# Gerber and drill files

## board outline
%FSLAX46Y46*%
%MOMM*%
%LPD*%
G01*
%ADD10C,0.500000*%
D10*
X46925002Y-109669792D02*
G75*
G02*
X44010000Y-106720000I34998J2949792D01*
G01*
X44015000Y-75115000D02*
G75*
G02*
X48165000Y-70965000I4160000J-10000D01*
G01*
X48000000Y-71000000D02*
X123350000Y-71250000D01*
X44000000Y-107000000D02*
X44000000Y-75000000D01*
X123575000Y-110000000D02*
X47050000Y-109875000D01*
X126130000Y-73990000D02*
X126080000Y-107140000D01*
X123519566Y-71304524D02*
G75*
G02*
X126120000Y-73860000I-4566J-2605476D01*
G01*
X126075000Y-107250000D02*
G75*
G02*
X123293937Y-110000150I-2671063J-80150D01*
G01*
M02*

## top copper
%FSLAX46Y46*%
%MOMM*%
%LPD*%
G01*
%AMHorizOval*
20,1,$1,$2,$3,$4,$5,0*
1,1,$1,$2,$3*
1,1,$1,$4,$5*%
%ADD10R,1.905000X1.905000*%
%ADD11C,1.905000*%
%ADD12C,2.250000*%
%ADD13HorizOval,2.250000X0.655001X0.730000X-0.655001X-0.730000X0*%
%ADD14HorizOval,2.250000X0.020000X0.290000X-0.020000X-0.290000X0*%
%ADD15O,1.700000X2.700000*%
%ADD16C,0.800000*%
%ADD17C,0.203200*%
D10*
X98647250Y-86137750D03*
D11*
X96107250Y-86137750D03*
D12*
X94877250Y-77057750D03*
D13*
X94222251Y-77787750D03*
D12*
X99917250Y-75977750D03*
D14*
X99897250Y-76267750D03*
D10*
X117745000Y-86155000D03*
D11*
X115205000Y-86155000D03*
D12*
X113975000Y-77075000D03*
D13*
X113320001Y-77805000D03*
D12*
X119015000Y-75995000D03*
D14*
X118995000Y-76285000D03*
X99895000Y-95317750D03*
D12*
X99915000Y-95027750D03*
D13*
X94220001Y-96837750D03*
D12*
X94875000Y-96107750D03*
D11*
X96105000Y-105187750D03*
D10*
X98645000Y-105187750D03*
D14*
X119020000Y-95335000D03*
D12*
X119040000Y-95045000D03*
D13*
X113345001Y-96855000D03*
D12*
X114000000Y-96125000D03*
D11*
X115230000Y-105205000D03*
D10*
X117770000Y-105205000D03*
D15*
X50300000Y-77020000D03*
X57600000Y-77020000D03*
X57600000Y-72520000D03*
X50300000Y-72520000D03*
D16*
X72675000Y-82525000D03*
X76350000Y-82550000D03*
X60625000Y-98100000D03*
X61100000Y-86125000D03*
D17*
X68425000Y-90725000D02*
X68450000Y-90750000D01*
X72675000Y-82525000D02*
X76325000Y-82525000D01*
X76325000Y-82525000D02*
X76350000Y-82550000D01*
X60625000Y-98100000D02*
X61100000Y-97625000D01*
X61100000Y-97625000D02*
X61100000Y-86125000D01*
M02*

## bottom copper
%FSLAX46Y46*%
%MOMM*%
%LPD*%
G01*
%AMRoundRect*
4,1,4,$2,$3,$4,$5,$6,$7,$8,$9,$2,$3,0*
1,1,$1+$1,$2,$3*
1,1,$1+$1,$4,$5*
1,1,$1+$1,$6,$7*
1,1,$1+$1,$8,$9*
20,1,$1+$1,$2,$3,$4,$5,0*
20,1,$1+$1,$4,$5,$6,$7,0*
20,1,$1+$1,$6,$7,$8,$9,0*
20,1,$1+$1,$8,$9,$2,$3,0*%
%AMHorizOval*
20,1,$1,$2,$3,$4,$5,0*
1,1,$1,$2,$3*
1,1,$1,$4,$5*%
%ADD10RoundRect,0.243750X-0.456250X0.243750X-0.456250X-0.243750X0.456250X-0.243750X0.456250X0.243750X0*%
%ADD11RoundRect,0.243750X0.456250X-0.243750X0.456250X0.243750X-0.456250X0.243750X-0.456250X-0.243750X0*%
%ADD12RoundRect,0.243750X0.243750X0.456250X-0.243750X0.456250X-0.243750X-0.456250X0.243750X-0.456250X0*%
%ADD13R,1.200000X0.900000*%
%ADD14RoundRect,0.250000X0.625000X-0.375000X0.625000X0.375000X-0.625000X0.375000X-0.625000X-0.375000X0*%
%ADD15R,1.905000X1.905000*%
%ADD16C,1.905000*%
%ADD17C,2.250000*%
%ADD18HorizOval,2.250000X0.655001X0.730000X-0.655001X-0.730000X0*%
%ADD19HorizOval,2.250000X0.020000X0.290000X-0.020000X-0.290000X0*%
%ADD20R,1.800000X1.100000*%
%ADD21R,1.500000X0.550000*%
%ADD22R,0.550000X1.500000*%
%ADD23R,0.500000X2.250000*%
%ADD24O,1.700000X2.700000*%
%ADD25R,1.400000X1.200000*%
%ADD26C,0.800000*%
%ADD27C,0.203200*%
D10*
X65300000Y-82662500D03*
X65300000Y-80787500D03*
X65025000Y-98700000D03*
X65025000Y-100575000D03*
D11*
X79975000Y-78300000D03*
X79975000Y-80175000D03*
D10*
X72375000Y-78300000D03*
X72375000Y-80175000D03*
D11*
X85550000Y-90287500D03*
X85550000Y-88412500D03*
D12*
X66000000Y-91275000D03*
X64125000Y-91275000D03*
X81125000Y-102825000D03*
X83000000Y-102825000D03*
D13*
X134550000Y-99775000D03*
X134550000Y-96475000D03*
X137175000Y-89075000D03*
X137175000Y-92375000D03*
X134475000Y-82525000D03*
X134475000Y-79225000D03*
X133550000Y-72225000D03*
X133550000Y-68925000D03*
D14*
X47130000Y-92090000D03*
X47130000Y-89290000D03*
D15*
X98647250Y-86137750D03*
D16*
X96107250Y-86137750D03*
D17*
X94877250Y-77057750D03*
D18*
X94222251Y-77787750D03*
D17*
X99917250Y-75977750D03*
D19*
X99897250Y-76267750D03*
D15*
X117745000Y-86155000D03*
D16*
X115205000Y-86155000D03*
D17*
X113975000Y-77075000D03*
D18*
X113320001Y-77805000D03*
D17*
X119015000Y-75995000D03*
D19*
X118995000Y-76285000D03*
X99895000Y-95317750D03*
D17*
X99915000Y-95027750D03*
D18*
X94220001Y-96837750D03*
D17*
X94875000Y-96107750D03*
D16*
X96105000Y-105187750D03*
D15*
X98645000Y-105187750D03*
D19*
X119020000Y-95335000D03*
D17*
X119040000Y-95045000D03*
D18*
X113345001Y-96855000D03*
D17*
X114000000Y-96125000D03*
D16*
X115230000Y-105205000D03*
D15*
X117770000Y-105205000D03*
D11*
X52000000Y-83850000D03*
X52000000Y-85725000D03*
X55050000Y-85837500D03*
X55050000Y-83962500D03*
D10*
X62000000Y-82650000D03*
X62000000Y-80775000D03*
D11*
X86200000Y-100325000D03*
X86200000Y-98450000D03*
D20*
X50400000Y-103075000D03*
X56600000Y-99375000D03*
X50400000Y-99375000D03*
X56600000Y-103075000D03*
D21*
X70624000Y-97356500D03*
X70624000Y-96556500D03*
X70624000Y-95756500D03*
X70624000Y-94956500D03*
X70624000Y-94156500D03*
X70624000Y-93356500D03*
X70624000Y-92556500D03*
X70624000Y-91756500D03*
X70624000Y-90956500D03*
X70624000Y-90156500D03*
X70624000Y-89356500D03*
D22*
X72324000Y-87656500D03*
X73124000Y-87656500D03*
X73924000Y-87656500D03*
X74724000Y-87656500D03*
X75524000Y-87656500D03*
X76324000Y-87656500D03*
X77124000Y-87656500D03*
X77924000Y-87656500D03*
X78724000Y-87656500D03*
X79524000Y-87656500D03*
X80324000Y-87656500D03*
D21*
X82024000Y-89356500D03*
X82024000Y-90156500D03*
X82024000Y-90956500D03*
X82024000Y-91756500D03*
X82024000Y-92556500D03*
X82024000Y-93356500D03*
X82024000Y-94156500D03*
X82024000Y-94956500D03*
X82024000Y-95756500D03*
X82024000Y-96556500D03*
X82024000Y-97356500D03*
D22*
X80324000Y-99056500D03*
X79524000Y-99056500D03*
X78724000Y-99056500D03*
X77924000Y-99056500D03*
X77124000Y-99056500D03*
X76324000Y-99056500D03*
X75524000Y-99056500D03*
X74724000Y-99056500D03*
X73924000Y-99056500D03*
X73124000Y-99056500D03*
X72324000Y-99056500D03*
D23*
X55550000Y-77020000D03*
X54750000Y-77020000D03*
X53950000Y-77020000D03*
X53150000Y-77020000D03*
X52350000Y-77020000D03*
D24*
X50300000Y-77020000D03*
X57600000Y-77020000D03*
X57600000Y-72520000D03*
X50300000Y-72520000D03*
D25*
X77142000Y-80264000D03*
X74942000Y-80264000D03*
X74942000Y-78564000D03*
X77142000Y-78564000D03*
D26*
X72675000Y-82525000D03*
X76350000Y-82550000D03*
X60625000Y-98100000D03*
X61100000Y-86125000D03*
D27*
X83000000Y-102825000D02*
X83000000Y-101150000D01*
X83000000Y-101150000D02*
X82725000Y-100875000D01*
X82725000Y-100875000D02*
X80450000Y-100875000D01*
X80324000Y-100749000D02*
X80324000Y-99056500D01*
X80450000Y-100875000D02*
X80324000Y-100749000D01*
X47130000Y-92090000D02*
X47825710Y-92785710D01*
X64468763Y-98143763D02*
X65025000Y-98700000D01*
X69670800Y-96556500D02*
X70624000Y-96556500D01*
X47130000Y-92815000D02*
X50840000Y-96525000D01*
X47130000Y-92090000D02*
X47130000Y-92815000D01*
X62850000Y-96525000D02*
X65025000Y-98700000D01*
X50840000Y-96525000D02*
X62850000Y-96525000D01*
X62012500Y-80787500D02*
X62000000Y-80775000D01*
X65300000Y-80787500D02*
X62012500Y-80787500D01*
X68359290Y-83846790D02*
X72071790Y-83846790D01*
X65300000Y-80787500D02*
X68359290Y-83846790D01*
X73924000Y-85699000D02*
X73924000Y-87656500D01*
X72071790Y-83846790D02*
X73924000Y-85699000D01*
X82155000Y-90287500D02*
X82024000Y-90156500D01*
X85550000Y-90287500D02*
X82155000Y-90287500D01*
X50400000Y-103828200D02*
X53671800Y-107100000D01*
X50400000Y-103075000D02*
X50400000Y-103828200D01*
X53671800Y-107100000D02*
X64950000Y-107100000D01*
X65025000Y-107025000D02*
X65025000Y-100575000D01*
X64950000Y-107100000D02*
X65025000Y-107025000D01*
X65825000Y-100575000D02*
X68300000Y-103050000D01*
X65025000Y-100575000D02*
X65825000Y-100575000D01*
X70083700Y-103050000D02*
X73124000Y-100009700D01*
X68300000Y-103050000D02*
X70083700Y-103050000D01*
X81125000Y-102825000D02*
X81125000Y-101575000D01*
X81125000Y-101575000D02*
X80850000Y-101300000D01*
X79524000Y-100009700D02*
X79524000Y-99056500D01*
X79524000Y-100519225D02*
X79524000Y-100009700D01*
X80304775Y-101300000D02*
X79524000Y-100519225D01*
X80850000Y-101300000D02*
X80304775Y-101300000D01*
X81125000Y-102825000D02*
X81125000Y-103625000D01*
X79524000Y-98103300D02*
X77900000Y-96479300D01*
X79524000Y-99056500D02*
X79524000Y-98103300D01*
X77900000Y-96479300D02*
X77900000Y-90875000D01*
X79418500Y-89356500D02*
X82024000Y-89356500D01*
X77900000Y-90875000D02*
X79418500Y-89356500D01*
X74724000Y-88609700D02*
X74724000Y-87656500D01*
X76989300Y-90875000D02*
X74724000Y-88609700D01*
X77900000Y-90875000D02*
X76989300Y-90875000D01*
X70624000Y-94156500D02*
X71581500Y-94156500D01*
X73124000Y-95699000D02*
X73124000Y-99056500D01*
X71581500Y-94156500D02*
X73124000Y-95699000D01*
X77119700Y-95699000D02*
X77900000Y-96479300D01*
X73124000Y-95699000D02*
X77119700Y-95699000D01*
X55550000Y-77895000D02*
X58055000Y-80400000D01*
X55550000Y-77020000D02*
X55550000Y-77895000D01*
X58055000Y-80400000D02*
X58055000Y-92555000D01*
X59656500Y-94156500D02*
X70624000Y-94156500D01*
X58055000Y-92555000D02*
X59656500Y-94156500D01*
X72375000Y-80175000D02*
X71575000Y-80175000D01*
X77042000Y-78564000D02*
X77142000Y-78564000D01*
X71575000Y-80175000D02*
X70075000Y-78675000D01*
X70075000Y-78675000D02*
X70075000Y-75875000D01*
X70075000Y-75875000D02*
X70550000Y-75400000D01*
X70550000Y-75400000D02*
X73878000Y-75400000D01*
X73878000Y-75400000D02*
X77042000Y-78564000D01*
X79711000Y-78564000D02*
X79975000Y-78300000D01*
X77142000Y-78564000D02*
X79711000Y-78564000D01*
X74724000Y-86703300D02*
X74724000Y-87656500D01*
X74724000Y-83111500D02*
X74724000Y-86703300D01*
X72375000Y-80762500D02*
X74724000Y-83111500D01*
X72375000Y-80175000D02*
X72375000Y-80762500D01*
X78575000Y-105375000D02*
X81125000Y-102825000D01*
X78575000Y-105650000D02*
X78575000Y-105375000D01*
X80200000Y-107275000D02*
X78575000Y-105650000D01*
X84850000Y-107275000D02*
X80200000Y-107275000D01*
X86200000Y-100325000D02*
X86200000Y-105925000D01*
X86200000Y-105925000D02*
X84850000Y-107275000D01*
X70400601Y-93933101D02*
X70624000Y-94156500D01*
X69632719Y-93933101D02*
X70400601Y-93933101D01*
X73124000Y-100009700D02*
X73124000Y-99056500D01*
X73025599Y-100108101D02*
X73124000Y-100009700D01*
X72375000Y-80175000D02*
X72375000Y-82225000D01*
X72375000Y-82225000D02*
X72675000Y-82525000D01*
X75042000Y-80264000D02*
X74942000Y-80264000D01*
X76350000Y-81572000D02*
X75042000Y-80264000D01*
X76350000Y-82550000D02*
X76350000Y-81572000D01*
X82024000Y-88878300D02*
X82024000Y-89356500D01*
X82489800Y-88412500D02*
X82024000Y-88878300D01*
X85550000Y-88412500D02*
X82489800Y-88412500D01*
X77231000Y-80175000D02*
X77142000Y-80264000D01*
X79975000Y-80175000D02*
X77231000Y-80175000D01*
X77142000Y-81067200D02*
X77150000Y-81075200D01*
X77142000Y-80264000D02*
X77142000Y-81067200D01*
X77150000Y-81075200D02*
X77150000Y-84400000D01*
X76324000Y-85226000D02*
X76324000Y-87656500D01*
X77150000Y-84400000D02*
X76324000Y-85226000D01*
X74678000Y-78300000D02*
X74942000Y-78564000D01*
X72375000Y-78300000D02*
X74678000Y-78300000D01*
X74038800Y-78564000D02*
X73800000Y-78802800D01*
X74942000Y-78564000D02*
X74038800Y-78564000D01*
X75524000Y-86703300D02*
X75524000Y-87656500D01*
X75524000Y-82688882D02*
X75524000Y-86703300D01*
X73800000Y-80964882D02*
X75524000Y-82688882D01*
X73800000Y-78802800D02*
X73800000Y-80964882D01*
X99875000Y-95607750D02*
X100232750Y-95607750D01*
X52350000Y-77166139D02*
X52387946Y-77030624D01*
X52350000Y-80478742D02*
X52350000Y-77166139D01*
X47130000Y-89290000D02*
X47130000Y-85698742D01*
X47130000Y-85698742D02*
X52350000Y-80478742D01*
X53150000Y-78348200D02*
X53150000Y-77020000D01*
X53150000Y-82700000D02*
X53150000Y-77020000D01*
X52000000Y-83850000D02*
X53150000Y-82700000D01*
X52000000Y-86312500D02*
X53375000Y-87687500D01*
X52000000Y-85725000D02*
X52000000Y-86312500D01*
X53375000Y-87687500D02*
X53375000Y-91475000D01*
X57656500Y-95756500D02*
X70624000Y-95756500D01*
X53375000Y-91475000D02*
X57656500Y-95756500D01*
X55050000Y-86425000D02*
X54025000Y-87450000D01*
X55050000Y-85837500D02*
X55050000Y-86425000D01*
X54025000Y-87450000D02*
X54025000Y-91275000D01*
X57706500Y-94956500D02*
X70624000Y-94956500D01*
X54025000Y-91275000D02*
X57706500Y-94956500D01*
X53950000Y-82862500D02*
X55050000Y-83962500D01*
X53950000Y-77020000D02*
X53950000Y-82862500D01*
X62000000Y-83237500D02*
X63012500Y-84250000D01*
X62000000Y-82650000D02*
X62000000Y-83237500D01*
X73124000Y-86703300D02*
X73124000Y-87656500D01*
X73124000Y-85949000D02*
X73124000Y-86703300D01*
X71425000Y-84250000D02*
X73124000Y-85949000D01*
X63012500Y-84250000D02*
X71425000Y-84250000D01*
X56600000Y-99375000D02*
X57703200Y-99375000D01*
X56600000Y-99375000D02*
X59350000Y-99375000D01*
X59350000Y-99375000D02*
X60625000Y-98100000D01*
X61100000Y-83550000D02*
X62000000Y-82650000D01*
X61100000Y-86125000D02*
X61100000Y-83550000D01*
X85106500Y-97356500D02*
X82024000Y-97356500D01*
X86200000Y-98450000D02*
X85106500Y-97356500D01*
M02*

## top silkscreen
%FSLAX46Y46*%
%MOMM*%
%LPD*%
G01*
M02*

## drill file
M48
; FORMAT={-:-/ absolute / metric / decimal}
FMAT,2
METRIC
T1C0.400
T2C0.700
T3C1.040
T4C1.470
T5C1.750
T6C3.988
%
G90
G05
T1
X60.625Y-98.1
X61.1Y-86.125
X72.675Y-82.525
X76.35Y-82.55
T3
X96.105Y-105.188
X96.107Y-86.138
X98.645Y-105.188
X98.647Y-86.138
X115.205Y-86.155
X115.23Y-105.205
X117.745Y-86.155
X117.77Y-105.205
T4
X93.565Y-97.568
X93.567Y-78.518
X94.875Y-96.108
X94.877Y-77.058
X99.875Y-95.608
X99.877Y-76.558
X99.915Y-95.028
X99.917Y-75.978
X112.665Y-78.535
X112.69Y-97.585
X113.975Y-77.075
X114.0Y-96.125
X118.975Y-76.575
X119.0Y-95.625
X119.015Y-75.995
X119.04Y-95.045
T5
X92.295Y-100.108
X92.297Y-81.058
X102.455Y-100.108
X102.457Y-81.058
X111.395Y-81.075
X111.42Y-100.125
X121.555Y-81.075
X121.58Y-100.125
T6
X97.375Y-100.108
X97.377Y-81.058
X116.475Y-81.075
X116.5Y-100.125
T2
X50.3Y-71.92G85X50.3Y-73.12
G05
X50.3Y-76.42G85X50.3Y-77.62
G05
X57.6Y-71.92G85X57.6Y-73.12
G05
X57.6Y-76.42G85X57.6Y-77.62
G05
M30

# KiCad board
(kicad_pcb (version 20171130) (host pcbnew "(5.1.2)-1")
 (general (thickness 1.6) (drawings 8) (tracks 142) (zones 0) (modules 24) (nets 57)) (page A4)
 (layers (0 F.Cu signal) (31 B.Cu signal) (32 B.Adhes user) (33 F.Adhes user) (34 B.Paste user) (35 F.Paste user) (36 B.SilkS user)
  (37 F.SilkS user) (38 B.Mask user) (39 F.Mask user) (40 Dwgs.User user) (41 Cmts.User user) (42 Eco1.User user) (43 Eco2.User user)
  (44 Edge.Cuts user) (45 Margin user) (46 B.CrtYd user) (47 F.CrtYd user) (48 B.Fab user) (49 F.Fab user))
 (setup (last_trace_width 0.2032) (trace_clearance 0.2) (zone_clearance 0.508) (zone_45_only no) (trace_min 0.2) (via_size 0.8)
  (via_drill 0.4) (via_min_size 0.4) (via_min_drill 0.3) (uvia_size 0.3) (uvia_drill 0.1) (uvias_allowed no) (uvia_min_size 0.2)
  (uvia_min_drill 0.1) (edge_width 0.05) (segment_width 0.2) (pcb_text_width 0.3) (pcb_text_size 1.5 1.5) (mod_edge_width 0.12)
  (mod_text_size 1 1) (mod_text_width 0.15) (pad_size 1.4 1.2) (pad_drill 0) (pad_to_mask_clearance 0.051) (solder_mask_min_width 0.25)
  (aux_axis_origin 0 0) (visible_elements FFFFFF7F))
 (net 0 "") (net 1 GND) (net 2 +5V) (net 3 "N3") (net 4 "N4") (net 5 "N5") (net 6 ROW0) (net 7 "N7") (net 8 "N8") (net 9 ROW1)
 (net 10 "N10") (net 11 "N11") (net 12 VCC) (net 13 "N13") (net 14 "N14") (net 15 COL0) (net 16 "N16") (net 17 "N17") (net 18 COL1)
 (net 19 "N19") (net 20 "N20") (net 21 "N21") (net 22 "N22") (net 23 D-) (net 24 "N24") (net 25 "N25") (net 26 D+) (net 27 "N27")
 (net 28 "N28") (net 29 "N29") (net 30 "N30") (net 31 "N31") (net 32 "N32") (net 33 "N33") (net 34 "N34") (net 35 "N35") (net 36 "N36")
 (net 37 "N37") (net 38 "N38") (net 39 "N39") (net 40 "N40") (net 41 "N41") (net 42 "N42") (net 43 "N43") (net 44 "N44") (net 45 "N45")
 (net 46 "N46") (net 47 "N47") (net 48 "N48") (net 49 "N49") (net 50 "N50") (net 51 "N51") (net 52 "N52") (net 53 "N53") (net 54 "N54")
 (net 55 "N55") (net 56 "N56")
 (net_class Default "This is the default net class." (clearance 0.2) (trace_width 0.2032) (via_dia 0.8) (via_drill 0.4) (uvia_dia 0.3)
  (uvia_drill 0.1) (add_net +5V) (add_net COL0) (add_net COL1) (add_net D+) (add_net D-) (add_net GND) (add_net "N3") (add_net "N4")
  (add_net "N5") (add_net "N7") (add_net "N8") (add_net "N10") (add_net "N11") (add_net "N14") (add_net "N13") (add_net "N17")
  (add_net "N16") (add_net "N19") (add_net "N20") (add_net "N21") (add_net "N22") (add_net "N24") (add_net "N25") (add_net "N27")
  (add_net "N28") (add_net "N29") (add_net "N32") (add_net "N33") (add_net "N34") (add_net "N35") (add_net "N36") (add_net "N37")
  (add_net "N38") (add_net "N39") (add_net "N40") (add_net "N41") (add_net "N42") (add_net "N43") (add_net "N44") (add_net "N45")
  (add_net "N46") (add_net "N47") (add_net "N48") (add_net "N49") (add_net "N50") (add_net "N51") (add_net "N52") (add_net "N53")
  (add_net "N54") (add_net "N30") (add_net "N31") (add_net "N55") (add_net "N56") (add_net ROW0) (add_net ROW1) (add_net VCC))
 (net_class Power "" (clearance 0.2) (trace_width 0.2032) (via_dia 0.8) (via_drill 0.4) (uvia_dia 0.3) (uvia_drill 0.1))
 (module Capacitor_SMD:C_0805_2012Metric (layer B.Cu) (at 65.3 81.725 270)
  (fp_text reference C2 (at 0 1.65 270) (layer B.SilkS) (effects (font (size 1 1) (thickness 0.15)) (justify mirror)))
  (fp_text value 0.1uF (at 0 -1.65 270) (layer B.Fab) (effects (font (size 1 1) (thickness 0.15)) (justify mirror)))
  (pad 2 smd roundrect (at 0.9375 0 270) (size 0.975 1.4) (layers B.Cu B.Paste B.Mask) (roundrect_rratio 0.25) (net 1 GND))
  (pad 1 smd roundrect (at -0.9375 0 270) (size 0.975 1.4) (layers B.Cu B.Paste B.Mask) (roundrect_rratio 0.25) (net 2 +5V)))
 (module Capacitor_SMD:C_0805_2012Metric (layer B.Cu) (at 65.025 99.6375 270)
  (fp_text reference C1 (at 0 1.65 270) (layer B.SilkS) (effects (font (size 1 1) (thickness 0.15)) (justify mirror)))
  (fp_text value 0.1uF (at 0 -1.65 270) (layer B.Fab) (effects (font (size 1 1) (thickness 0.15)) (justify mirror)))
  (pad 1 smd roundrect (at -0.9375 0 270) (size 0.975 1.4) (layers B.Cu B.Paste B.Mask) (roundrect_rratio 0.25) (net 2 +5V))
  (pad 2 smd roundrect (at 0.9375 0 270) (size 0.975 1.4) (layers B.Cu B.Paste B.Mask) (roundrect_rratio 0.25) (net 1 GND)))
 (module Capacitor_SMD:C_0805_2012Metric (layer B.Cu) (at 79.975 79.2375 90)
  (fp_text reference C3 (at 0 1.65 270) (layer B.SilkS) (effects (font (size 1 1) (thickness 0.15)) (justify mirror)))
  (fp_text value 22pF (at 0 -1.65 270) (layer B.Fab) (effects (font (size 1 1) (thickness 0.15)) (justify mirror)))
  (pad 2 smd roundrect (at 0.9375 0 90) (size 0.975 1.4) (layers B.Cu B.Paste B.Mask) (roundrect_rratio 0.25) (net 1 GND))
  (pad 1 smd roundrect (at -0.9375 0 90) (size 0.975 1.4) (layers B.Cu B.Paste B.Mask) (roundrect_rratio 0.25) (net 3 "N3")))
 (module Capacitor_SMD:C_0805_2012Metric (layer B.Cu) (at 72.375 79.2375 270)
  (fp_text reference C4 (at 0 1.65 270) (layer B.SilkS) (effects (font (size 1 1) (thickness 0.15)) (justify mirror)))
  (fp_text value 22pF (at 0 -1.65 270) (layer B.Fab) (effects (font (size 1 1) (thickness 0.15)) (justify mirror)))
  (pad 1 smd roundrect (at -0.9375 0 270) (size 0.975 1.4) (layers B.Cu B.Paste B.Mask) (roundrect_rratio 0.25) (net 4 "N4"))
  (pad 2 smd roundrect (at 0.9375 0 270) (size 0.975 1.4) (layers B.Cu B.Paste B.Mask) (roundrect_rratio 0.25) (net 1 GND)))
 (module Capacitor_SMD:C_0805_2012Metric (layer B.Cu) (at 85.55 89.35 90)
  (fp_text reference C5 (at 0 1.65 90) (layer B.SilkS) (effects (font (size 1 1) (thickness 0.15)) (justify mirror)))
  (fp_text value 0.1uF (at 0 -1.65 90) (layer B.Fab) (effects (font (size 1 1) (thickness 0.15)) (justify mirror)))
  (pad 1 smd roundrect (at -0.9375 0 90) (size 0.975 1.4) (layers B.Cu B.Paste B.Mask) (roundrect_rratio 0.25) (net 2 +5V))
  (pad 2 smd roundrect (at 0.9375 0 90) (size 0.975 1.4) (layers B.Cu B.Paste B.Mask) (roundrect_rratio 0.25) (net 1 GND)))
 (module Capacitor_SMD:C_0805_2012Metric (layer B.Cu) (at 65.0625 91.275 180)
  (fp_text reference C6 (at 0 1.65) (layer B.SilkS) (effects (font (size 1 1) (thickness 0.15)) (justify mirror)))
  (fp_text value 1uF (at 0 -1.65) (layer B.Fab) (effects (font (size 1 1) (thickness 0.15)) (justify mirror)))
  (pad 1 smd roundrect (at -0.9375 0 180) (size 0.975 1.4) (layers B.Cu B.Paste B.Mask) (roundrect_rratio 0.25) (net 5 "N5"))
  (pad 2 smd roundrect (at 0.9375 0 180) (size 0.975 1.4) (layers B.Cu B.Paste B.Mask) (roundrect_rratio 0.25) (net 1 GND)))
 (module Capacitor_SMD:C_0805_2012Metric (layer B.Cu) (at 82.0625 102.825 180)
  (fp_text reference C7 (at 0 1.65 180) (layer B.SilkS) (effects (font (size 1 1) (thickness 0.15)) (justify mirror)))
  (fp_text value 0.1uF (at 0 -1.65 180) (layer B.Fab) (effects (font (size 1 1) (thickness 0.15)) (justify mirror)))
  (pad 2 smd roundrect (at 0.9375 0 180) (size 0.975 1.4) (layers B.Cu B.Paste B.Mask) (roundrect_rratio 0.25) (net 1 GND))
  (pad 1 smd roundrect (at -0.9375 0 180) (size 0.975 1.4) (layers B.Cu B.Paste B.Mask) (roundrect_rratio 0.25) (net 2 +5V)))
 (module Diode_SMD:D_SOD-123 (layer B.Cu) (at 134.55 98.125 90)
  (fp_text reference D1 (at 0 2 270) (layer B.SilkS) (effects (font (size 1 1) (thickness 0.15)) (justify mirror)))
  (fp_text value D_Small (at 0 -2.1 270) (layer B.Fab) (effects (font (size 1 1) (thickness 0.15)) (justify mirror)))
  (pad 1 smd rect (at -1.65 0 90) (size 0.9 1.2) (layers B.Cu B.Paste B.Mask) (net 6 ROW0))
  (pad 2 smd rect (at 1.65 0 90) (size 0.9 1.2) (layers B.Cu B.Paste B.Mask) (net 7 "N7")))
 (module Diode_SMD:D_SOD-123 (layer B.Cu) (at 137.175 90.725 90)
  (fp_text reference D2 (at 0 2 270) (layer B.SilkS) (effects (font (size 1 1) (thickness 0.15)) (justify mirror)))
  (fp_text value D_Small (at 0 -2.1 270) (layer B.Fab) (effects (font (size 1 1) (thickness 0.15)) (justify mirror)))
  (pad 2 smd rect (at 1.65 0 90) (size 0.9 1.2) (layers B.Cu B.Paste B.Mask) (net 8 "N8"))
  (pad 1 smd rect (at -1.65 0 90) (size 0.9 1.2) (layers B.Cu B.Paste B.Mask) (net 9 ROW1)))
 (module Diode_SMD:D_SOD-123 (layer B.Cu) (at 134.475 80.875 90)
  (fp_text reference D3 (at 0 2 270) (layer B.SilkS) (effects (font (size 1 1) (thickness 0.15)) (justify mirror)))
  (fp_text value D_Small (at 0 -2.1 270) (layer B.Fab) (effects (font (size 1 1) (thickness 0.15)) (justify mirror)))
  (pad 1 smd rect (at -1.65 0 90) (size 0.9 1.2) (layers B.Cu B.Paste B.Mask) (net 6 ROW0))
  (pad 2 smd rect (at 1.65 0 90) (size 0.9 1.2) (layers B.Cu B.Paste B.Mask) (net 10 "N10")))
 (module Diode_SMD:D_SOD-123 (layer B.Cu) (at 133.55 70.575 270)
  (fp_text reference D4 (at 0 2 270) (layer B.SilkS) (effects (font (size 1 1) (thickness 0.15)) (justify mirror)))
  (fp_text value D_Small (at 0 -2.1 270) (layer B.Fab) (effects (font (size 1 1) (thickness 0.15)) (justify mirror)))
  (pad 2 smd rect (at 1.65 0 270) (size 0.9 1.2) (layers B.Cu B.Paste B.Mask) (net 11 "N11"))
  (pad 1 smd rect (at -1.65 0 270) (size 0.9 1.2) (layers B.Cu B.Paste B.Mask) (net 9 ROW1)))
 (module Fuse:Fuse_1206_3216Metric (layer B.Cu) (at 47.13 90.69 90)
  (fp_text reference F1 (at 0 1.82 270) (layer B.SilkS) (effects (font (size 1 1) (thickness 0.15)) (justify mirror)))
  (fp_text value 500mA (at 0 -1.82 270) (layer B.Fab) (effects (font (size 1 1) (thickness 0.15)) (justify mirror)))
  (pad 1 smd roundrect (at -1.4 0 90) (size 1.25 1.75) (layers B.Cu B.Paste B.Mask) (roundrect_rratio 0.2) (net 2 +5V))
  (pad 2 smd roundrect (at 1.4 0 90) (size 1.25 1.75) (layers B.Cu B.Paste B.Mask) (roundrect_rratio 0.2) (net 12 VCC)))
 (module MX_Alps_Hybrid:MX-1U (layer F.Cu) (at 97.37725 81.05775)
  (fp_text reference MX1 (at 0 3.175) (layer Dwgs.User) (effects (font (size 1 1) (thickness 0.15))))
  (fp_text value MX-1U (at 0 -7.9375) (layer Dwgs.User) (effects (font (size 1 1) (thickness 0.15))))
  (pad "" np_thru_hole circle (at 5.08 0 48.0996) (size 1.75 1.75) (drill 1.75) (layers *.Cu *.Mask))
  (pad "" np_thru_hole circle (at -5.08 0 48.0996) (size 1.75 1.75) (drill 1.75) (layers *.Cu *.Mask))
  (pad 4 thru_hole rect (at 1.27 5.08) (size 1.905 1.905) (drill 1.04) (layers *.Cu B.Mask) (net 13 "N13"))
  (pad 3 thru_hole circle (at -1.27 5.08) (size 1.905 1.905) (drill 1.04) (layers *.Cu B.Mask) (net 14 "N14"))
  (pad 1 thru_hole circle (at -2.5 -4) (size 2.25 2.25) (drill 1.47) (layers *.Cu B.Mask) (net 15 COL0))
  (pad "" np_thru_hole circle (at 0 0) (size 3.9878 3.9878) (drill 3.9878) (layers *.Cu *.Mask))
  (pad 1 thru_hole oval (at -3.81 -2.54 48.0996) (size 4.211556 2.25) (drill 1.47 (offset 0.980778 0)) (layers *.Cu B.Mask) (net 15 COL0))
  (pad 2 thru_hole circle (at 2.54 -5.08) (size 2.25 2.25) (drill 1.47) (layers *.Cu B.Mask) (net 7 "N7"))
  (pad 2 thru_hole oval (at 2.5 -4.5 86.0548) (size 2.831378 2.25) (drill 1.47 (offset 0.290689 0)) (layers *.Cu B.Mask) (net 7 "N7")))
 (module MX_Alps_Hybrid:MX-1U (layer F.Cu) (at 116.475 81.075)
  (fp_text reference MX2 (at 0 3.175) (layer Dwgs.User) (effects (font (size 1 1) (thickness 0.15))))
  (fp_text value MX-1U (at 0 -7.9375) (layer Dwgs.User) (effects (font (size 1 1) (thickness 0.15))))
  (pad "" np_thru_hole circle (at 5.08 0 48.0996) (size 1.75 1.75) (drill 1.75) (layers *.Cu *.Mask))
  (pad "" np_thru_hole circle (at -5.08 0 48.0996) (size 1.75 1.75) (drill 1.75) (layers *.Cu *.Mask))
  (pad 4 thru_hole rect (at 1.27 5.08) (size 1.905 1.905) (drill 1.04) (layers *.Cu B.Mask) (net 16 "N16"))
  (pad 3 thru_hole circle (at -1.27 5.08) (size 1.905 1.905) (drill 1.04) (layers *.Cu B.Mask) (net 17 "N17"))
  (pad 1 thru_hole circle (at -2.5 -4) (size 2.25 2.25) (drill 1.47) (layers *.Cu B.Mask) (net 15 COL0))
  (pad "" np_thru_hole circle (at 0 0) (size 3.9878 3.9878) (drill 3.9878) (layers *.Cu *.Mask))
  (pad 1 thru_hole oval (at -3.81 -2.54 48.0996) (size 4.211556 2.25) (drill 1.47 (offset 0.980778 0)) (layers *.Cu B.Mask) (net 15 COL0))
  (pad 2 thru_hole circle (at 2.54 -5.08) (size 2.25 2.25) (drill 1.47) (layers *.Cu B.Mask) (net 8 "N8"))
  (pad 2 thru_hole oval (at 2.5 -4.5 86.0548) (size 2.831378 2.25) (drill 1.47 (offset 0.290689 0)) (layers *.Cu B.Mask) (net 8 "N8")))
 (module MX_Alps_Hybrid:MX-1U (layer F.Cu) (at 97.375 100.10775)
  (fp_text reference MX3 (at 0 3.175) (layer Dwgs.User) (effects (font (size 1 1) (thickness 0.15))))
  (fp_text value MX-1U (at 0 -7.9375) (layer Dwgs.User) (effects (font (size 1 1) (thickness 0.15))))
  (pad 2 thru_hole oval (at 2.5 -4.5 86.0548) (size 2.831378 2.25) (drill 1.47 (offset 0.290689 0)) (layers *.Cu B.Mask) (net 10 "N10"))
  (pad 2 thru_hole circle (at 2.54 -5.08) (size 2.25 2.25) (drill 1.47) (layers *.Cu B.Mask) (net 10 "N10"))
  (pad 1 thru_hole oval (at -3.81 -2.54 48.0996) (size 4.211556 2.25) (drill 1.47 (offset 0.980778 0)) (layers *.Cu B.Mask) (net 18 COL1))
  (pad "" np_thru_hole circle (at 0 0) (size 3.9878 3.9878) (drill 3.9878) (layers *.Cu *.Mask))
  (pad 1 thru_hole circle (at -2.5 -4) (size 2.25 2.25) (drill 1.47) (layers *.Cu B.Mask) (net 18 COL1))
  (pad 3 thru_hole circle (at -1.27 5.08) (size 1.905 1.905) (drill 1.04) (layers *.Cu B.Mask) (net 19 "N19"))
  (pad 4 thru_hole rect (at 1.27 5.08) (size 1.905 1.905) (drill 1.04) (layers *.Cu B.Mask) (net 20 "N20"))
  (pad "" np_thru_hole circle (at -5.08 0 48.0996) (size 1.75 1.75) (drill 1.75) (layers *.Cu *.Mask))
  (pad "" np_thru_hole circle (at 5.08 0 48.0996) (size 1.75 1.75) (drill 1.75) (layers *.Cu *.Mask)))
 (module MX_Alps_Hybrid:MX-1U (layer F.Cu) (at 116.5 100.125)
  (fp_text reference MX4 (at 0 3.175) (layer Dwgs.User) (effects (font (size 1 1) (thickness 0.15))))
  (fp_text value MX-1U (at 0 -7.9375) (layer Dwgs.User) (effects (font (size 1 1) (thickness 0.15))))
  (pad 2 thru_hole oval (at 2.5 -4.5 86.0548) (size 2.831378 2.25) (drill 1.47 (offset 0.290689 0)) (layers *.Cu B.Mask) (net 11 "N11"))
  (pad 2 thru_hole circle (at 2.54 -5.08) (size 2.25 2.25) (drill 1.47) (layers *.Cu B.Mask) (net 11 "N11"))
  (pad 1 thru_hole oval (at -3.81 -2.54 48.0996) (size 4.211556 2.25) (drill 1.47 (offset 0.980778 0)) (layers *.Cu B.Mask) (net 18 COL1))
  (pad "" np_thru_hole circle (at 0 0) (size 3.9878 3.9878) (drill 3.9878) (layers *.Cu *.Mask))
  (pad 1 thru_hole circle (at -2.5 -4) (size 2.25 2.25) (drill 1.47) (layers *.Cu B.Mask) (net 18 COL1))
  (pad 3 thru_hole circle (at -1.27 5.08) (size 1.905 1.905) (drill 1.04) (layers *.Cu B.Mask) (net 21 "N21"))
  (pad 4 thru_hole rect (at 1.27 5.08) (size 1.905 1.905) (drill 1.04) (layers *.Cu B.Mask) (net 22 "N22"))
  (pad "" np_thru_hole circle (at -5.08 0 48.0996) (size 1.75 1.75) (drill 1.75) (layers *.Cu *.Mask))
  (pad "" np_thru_hole circle (at 5.08 0 48.0996) (size 1.75 1.75) (drill 1.75) (layers *.Cu *.Mask)))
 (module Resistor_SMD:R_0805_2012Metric (layer B.Cu) (at 52 84.7875 90)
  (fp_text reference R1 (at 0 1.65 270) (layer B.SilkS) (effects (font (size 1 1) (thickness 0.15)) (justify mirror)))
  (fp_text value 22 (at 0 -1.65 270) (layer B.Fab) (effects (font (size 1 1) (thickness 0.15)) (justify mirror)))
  (pad 2 smd roundrect (at 0.9375 0 90) (size 0.975 1.4) (layers B.Cu B.Paste B.Mask) (roundrect_rratio 0.25) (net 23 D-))
  (pad 1 smd roundrect (at -0.9375 0 90) (size 0.975 1.4) (layers B.Cu B.Paste B.Mask) (roundrect_rratio 0.25) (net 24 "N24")))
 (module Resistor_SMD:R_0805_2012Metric (layer B.Cu) (at 55.05 84.9 90)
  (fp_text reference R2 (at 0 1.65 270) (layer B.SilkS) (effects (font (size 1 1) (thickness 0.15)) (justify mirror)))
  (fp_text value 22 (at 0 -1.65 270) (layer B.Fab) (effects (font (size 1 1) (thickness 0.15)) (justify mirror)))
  (pad 1 smd roundrect (at -0.9375 0 90) (size 0.975 1.4) (layers B.Cu B.Paste B.Mask) (roundrect_rratio 0.25) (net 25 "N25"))
  (pad 2 smd roundrect (at 0.9375 0 90) (size 0.975 1.4) (layers B.Cu B.Paste B.Mask) (roundrect_rratio 0.25) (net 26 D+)))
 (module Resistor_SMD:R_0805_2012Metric (layer B.Cu) (at 62 81.7125 270)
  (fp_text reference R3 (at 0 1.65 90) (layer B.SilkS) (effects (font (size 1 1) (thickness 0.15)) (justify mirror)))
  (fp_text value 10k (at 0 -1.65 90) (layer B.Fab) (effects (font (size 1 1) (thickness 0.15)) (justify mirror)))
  (pad 2 smd roundrect (at 0.9375 0 270) (size 0.975 1.4) (layers B.Cu B.Paste B.Mask) (roundrect_rratio 0.25) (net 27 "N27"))
  (pad 1 smd roundrect (at -0.9375 0 270) (size 0.975 1.4) (layers B.Cu B.Paste B.Mask) (roundrect_rratio 0.25) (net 2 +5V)))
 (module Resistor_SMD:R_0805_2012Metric (layer B.Cu) (at 86.2 99.3875 90)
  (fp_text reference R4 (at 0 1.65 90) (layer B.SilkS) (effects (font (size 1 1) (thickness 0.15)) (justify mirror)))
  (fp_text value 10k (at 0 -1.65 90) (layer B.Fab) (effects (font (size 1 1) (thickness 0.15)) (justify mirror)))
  (pad 1 smd roundrect (at -0.9375 0 90) (size 0.975 1.4) (layers B.Cu B.Paste B.Mask) (roundrect_rratio 0.25) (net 1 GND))
  (pad 2 smd roundrect (at 0.9375 0 90) (size 0.975 1.4) (layers B.Cu B.Paste B.Mask) (roundrect_rratio 0.25) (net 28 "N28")))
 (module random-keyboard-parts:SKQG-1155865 (layer B.Cu) (at 53.5 101.225 180)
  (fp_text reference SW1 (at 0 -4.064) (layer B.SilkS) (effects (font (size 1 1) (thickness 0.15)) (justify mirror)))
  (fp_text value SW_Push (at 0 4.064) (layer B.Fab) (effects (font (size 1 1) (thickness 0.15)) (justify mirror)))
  (pad 1 smd rect (at 3.1 -1.85 180) (size 1.8 1.1) (layers B.Cu B.Paste B.Mask) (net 1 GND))
  (pad 2 smd rect (at -3.1 1.85 180) (size 1.8 1.1) (layers B.Cu B.Paste B.Mask) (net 27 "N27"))
  (pad 3 smd rect (at 3.1 1.85 180) (size 1.8 1.1) (layers B.Cu B.Paste B.Mask))
  (pad 4 smd rect (at -3.1 -1.85 180) (size 1.8 1.1) (layers B.Cu B.Paste B.Mask)))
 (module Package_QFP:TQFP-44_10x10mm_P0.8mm (layer B.Cu) (at 76.324 93.3565)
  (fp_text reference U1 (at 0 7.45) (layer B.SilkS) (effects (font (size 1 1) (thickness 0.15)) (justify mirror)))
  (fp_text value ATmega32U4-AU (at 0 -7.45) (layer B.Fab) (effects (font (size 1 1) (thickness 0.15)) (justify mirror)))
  (pad 1 smd rect (at -5.7 4) (size 1.5 0.55) (layers B.Cu B.Paste B.Mask) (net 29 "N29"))
  (pad 2 smd rect (at -5.7 3.2) (size 1.5 0.55) (layers B.Cu B.Paste B.Mask) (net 2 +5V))
  (pad 3 smd rect (at -5.7 2.4) (size 1.5 0.55) (layers B.Cu B.Paste B.Mask) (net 24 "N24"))
  (pad 4 smd rect (at -5.7 1.6) (size 1.5 0.55) (layers B.Cu B.Paste B.Mask) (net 25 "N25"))
  (pad 5 smd rect (at -5.7 0.8) (size 1.5 0.55) (layers B.Cu B.Paste B.Mask) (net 1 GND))
  (pad 6 smd rect (at -5.7 0) (size 1.5 0.55) (layers B.Cu B.Paste B.Mask) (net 5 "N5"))
  (pad 7 smd rect (at -5.7 -0.8) (size 1.5 0.55) (layers B.Cu B.Paste B.Mask) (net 2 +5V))
  (pad 8 smd rect (at -5.7 -1.6) (size 1.5 0.55) (layers B.Cu B.Paste B.Mask) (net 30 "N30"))
  (pad 9 smd rect (at -5.7 -2.4) (size 1.5 0.55) (layers B.Cu B.Paste B.Mask) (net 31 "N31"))
  (pad 10 smd rect (at -5.7 -3.2) (size 1.5 0.55) (layers B.Cu B.Paste B.Mask) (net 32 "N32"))
  (pad 11 smd rect (at -5.7 -4) (size 1.5 0.55) (layers B.Cu B.Paste B.Mask) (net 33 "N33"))
  (pad 12 smd rect (at -4 -5.7 270) (size 1.5 0.55) (layers B.Cu B.Paste B.Mask) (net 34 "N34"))
  (pad 13 smd rect (at -3.2 -5.7 270) (size 1.5 0.55) (layers B.Cu B.Paste B.Mask) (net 27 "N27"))
  (pad 14 smd rect (at -2.4 -5.7 270) (size 1.5 0.55) (layers B.Cu B.Paste B.Mask) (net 2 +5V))
  (pad 15 smd rect (at -1.6 -5.7 270) (size 1.5 0.55) (layers B.Cu B.Paste B.Mask) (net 1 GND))
  (pad 16 smd rect (at -0.8 -5.7 270) (size 1.5 0.55) (layers B.Cu B.Paste B.Mask) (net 4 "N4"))
  (pad 17 smd rect (at 0 -5.7 270) (size 1.5 0.55) (layers B.Cu B.Paste B.Mask) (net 3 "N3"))
  (pad 18 smd rect (at 0.8 -5.7 270) (size 1.5 0.55) (layers B.Cu B.Paste B.Mask) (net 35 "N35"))
  (pad 19 smd rect (at 1.6 -5.7 270) (size 1.5 0.55) (layers B.Cu B.Paste B.Mask) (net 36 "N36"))
  (pad 20 smd rect (at 2.4 -5.7 270) (size 1.5 0.55) (layers B.Cu B.Paste B.Mask) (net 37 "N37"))
  (pad 21 smd rect (at 3.2 -5.7 270) (size 1.5 0.55) (layers B.Cu B.Paste B.Mask) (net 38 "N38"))
  (pad 22 smd rect (at 4 -5.7 270) (size 1.5 0.55) (layers B.Cu B.Paste B.Mask) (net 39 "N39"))
  (pad 23 smd rect (at 5.7 -4) (size 1.5 0.55) (layers B.Cu B.Paste B.Mask) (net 1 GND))
  (pad 24 smd rect (at 5.7 -3.2) (size 1.5 0.55) (layers B.Cu B.Paste B.Mask) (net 2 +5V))
  (pad 25 smd rect (at 5.7 -2.4) (size 1.5 0.55) (layers B.Cu B.Paste B.Mask) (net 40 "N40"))
  (pad 26 smd rect (at 5.7 -1.6) (size 1.5 0.55) (layers B.Cu B.Paste B.Mask) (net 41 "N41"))
  (pad 27 smd rect (at 5.7 -0.8) (size 1.5 0.55) (layers B.Cu B.Paste B.Mask) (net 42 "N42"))
  (pad 28 smd rect (at 5.7 0) (size 1.5 0.55) (layers B.Cu B.Paste B.Mask) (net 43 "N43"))
  (pad 29 smd rect (at 5.7 0.8) (size 1.5 0.55) (layers B.Cu B.Paste B.Mask) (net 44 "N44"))
  (pad 30 smd rect (at 5.7 1.6) (size 1.5 0.55) (layers B.Cu B.Paste B.Mask) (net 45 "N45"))
  (pad 31 smd rect (at 5.7 2.4) (size 1.5 0.55) (layers B.Cu B.Paste B.Mask) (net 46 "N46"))
  (pad 32 smd rect (at 5.7 3.2) (size 1.5 0.55) (layers B.Cu B.Paste B.Mask) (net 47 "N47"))
  (pad 33 smd rect (at 5.7 4) (size 1.5 0.55) (layers B.Cu B.Paste B.Mask) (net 28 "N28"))
  (pad 34 smd rect (at 4 5.7 270) (size 1.5 0.55) (layers B.Cu B.Paste B.Mask) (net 2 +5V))
  (pad 35 smd rect (at 3.2 5.7 270) (size 1.5 0.55) (layers B.Cu B.Paste B.Mask) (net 1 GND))
  (pad 36 smd rect (at 2.4 5.7 270) (size 1.5 0.55) (layers B.Cu B.Paste B.Mask) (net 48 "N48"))
  (pad 37 smd rect (at 1.6 5.7 270) (size 1.5 0.55) (layers B.Cu B.Paste B.Mask) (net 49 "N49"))
  (pad 38 smd rect (at 0.8 5.7 270) (size 1.5 0.55) (layers B.Cu B.Paste B.Mask) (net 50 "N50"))
  (pad 39 smd rect (at 0 5.7 270) (size 1.5 0.55) (layers B.Cu B.Paste B.Mask) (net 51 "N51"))
  (pad 40 smd rect (at -0.8 5.7 270) (size 1.5 0.55) (layers B.Cu B.Paste B.Mask) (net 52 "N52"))
  (pad 41 smd rect (at -1.6 5.7 270) (size 1.5 0.55) (layers B.Cu B.Paste B.Mask) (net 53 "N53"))
  (pad 42 smd rect (at -2.4 5.7 270) (size 1.5 0.55) (layers B.Cu B.Paste B.Mask) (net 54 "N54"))
  (pad 43 smd rect (at -3.2 5.7 270) (size 1.5 0.55) (layers B.Cu B.Paste B.Mask) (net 1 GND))
  (pad 44 smd rect (at -4 5.7 270) (size 1.5 0.55) (layers B.Cu B.Paste B.Mask) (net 2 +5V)))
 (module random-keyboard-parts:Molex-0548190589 (layer B.Cu) (at 53.95 72.52 270)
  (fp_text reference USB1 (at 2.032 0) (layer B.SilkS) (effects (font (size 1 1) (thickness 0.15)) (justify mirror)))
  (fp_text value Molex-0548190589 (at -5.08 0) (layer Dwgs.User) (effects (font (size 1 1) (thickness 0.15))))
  (pad 1 smd rect (at 4.5 -1.6 270) (size 2.25 0.5) (layers B.Cu B.Paste B.Mask) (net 1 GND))
  (pad 2 smd rect (at 4.5 -0.8 270) (size 2.25 0.5) (layers B.Cu B.Paste B.Mask) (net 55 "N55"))
  (pad 3 smd rect (at 4.5 0 270) (size 2.25 0.5) (layers B.Cu B.Paste B.Mask) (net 26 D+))
  (pad 4 smd rect (at 4.5 0.8 270) (size 2.25 0.5) (layers B.Cu B.Paste B.Mask) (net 23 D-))
  (pad 5 smd rect (at 4.5 1.6 270) (size 2.25 0.5) (layers B.Cu B.Paste B.Mask) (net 12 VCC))
  (pad 6 thru_hole oval (at 4.5 3.65 270) (size 2.7 1.7) (drill oval 1.9 0.7) (layers *.Cu *.Mask) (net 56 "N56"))
  (pad 6 thru_hole oval (at 4.5 -3.65 270) (size 2.7 1.7) (drill oval 1.9 0.7) (layers *.Cu *.Mask) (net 56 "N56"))
  (pad 6 thru_hole oval (at 0 -3.65 270) (size 2.7 1.7) (drill oval 1.9 0.7) (layers *.Cu *.Mask) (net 56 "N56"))
  (pad 6 thru_hole oval (at 0 3.65 270) (size 2.7 1.7) (drill oval 1.9 0.7) (layers *.Cu *.Mask) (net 56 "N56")))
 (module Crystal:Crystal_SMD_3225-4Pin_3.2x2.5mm (layer B.Cu) (at 76.042 79.414 180)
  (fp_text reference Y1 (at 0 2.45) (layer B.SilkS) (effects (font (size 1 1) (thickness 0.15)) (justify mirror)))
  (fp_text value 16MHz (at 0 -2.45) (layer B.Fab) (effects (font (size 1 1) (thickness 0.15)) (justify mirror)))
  (pad 1 smd rect (at -1.1 -0.85 180) (size 1.4 1.2) (layers B.Cu B.Paste B.Mask) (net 3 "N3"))
  (pad 2 smd rect (at 1.1 -0.85 180) (size 1.4 1.2) (layers B.Cu B.Paste B.Mask) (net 1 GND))
  (pad 3 smd rect (at 1.1 0.85 180) (size 1.4 1.2) (layers B.Cu B.Paste B.Mask) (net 4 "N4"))
  (pad 4 smd rect (at -1.1 0.85 180) (size 1.4 1.2) (layers B.Cu B.Paste B.Mask) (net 1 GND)))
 (gr_arc (start 46.96 106.72) (end 44.01 106.72) (angle -89.32023579) (layer Edge.Cuts) (width 0.5))
 (gr_arc (start 48.175 75.125) (end 48.165 70.965) (angle -89.72454005) (layer Edge.Cuts) (width 0.5))
 (gr_line (start 48 71) (end 123.35 71.25) (layer Edge.Cuts) (width 0.5))
 (gr_line (start 44 107) (end 44 75) (layer Edge.Cuts) (width 0.5))
 (gr_line (start 123.575 110) (end 47.05 109.875) (layer Edge.Cuts) (width 0.5))
 (gr_line (start 126.13 73.99) (end 126.08 107.14) (layer Edge.Cuts) (width 0.5))
 (gr_arc (start 123.515 73.91) (end 126.12 73.86) (angle -88.8) (layer Edge.Cuts) (width 0.5))
 (gr_arc (start 123.403937 107.33015) (end 123.293937 110.00015) (angle -94.07790525) (layer Edge.Cuts) (width 0.5))
 (segment (start 83 102.825) (end 83 101.15) (width 0.2032) (layer B.Cu) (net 2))
 (segment (start 83 101.15) (end 82.725 100.875) (width 0.2032) (layer B.Cu) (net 2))
 (segment (start 82.725 100.875) (end 80.45 100.875) (width 0.2032) (layer B.Cu) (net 2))
 (segment (start 80.324 100.749) (end 80.324 99.0565) (width 0.2032) (layer B.Cu) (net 2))
 (segment (start 80.45 100.875) (end 80.324 100.749) (width 0.2032) (layer B.Cu) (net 2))
 (segment (start 47.13 92.09) (end 47.82571 92.78571) (width 0.2032) (layer B.Cu) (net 2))
 (segment (start 64.468763 98.143763) (end 65.025 98.7) (width 0.2032) (layer B.Cu) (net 2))
 (segment (start 69.6708 96.5565) (end 70.624 96.5565) (width 0.2032) (layer B.Cu) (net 2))
 (segment (start 47.13 92.815) (end 50.84 96.525) (width 0.2032) (layer B.Cu) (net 2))
 (segment (start 47.13 92.09) (end 47.13 92.815) (width 0.2032) (layer B.Cu) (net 2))
 (segment (start 62.85 96.525) (end 65.025 98.7) (width 0.2032) (layer B.Cu) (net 2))
 (segment (start 50.84 96.525) (end 62.85 96.525) (width 0.2032) (layer B.Cu) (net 2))
 (segment (start 62.0125 80.7875) (end 62 80.775) (width 0.2032) (layer B.Cu) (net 2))
 (segment (start 65.3 80.7875) (end 62.0125 80.7875) (width 0.2032) (layer B.Cu) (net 2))
 (segment (start 68.35929 83.84679) (end 72.07179 83.84679) (width 0.2032) (layer B.Cu) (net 2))
 (segment (start 65.3 80.7875) (end 68.35929 83.84679) (width 0.2032) (layer B.Cu) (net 2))
 (segment (start 73.924 85.699) (end 73.924 87.6565) (width 0.2032) (layer B.Cu) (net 2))
 (segment (start 72.07179 83.84679) (end 73.924 85.699) (width 0.2032) (layer B.Cu) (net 2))
 (segment (start 82.155 90.2875) (end 82.024 90.1565) (width 0.2032) (layer B.Cu) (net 2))
 (segment (start 85.55 90.2875) (end 82.155 90.2875) (width 0.2032) (layer B.Cu) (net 2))
 (segment (start 50.4 103.8282) (end 53.6718 107.1) (width 0.2032) (layer B.Cu) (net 1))
 (segment (start 50.4 103.075) (end 50.4 103.8282) (width 0.2032) (layer B.Cu) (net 1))
 (segment (start 53.6718 107.1) (end 64.95 107.1) (width 0.2032) (layer B.Cu) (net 1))
 (segment (start 65.025 107.025) (end 65.025 100.575) (width 0.2032) (layer B.Cu) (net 1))
 (segment (start 64.95 107.1) (end 65.025 107.025) (width 0.2032) (layer B.Cu) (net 1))
 (segment (start 65.825 100.575) (end 68.3 103.05) (width 0.2032) (layer B.Cu) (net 1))
 (segment (start 65.025 100.575) (end 65.825 100.575) (width 0.2032) (layer B.Cu) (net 1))
 (segment (start 70.0837 103.05) (end 73.124 100.0097) (width 0.2032) (layer B.Cu) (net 1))
 (segment (start 68.3 103.05) (end 70.0837 103.05) (width 0.2032) (layer B.Cu) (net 1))
 (segment (start 81.125 102.825) (end 81.125 101.575) (width 0.2032) (layer B.Cu) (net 1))
 (segment (start 81.125 101.575) (end 80.85 101.3) (width 0.2032) (layer B.Cu) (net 1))
 (segment (start 79.524 100.0097) (end 79.524 99.0565) (width 0.2032) (layer B.Cu) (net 1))
 (segment (start 79.524 100.519225) (end 79.524 100.0097) (width 0.2032) (layer B.Cu) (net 1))
 (segment (start 80.304775 101.3) (end 79.524 100.519225) (width 0.2032) (layer B.Cu) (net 1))
 (segment (start 80.85 101.3) (end 80.304775 101.3) (width 0.2032) (layer B.Cu) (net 1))
 (segment (start 81.125 102.825) (end 81.125 103.625) (width 0.2032) (layer B.Cu) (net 1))
 (segment (start 79.524 98.1033) (end 77.9 96.4793) (width 0.2032) (layer B.Cu) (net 1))
 (segment (start 79.524 99.0565) (end 79.524 98.1033) (width 0.2032) (layer B.Cu) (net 1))
 (segment (start 77.9 96.4793) (end 77.9 90.875) (width 0.2032) (layer B.Cu) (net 1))
 (segment (start 79.4185 89.3565) (end 82.024 89.3565) (width 0.2032) (layer B.Cu) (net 1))
 (segment (start 77.9 90.875) (end 79.4185 89.3565) (width 0.2032) (layer B.Cu) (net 1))
 (segment (start 74.724 88.6097) (end 74.724 87.6565) (width 0.2032) (layer B.Cu) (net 1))
 (segment (start 76.9893 90.875) (end 74.724 88.6097) (width 0.2032) (layer B.Cu) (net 1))
 (segment (start 77.9 90.875) (end 76.9893 90.875) (width 0.2032) (layer B.Cu) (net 1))
 (segment (start 70.624 94.1565) (end 71.5815 94.1565) (width 0.2032) (layer B.Cu) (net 1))
 (segment (start 73.124 95.699) (end 73.124 99.0565) (width 0.2032) (layer B.Cu) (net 1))
 (segment (start 71.5815 94.1565) (end 73.124 95.699) (width 0.2032) (layer B.Cu) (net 1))
 (segment (start 77.1197 95.699) (end 77.9 96.4793) (width 0.2032) (layer B.Cu) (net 1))
 (segment (start 73.124 95.699) (end 77.1197 95.699) (width 0.2032) (layer B.Cu) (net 1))
 (segment (start 55.55 77.895) (end 58.055 80.4) (width 0.2032) (layer B.Cu) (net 1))
 (segment (start 55.55 77.02) (end 55.55 77.895) (width 0.2032) (layer B.Cu) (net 1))
 (segment (start 58.055 80.4) (end 58.055 92.555) (width 0.2032) (layer B.Cu) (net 1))
 (segment (start 59.6565 94.1565) (end 70.624 94.1565) (width 0.2032) (layer B.Cu) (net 1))
 (segment (start 58.055 92.555) (end 59.6565 94.1565) (width 0.2032) (layer B.Cu) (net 1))
 (segment (start 72.375 80.175) (end 71.575 80.175) (width 0.2032) (layer B.Cu) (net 1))
 (segment (start 77.042 78.564) (end 77.142 78.564) (width 0.2032) (layer B.Cu) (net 1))
 (segment (start 71.575 80.175) (end 70.075 78.675) (width 0.2032) (layer B.Cu) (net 1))
 (segment (start 70.075 78.675) (end 70.075 75.875) (width 0.2032) (layer B.Cu) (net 1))
 (segment (start 70.075 75.875) (end 70.55 75.4) (width 0.2032) (layer B.Cu) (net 1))
 (segment (start 70.55 75.4) (end 73.878 75.4) (width 0.2032) (layer B.Cu) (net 1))
 (segment (start 73.878 75.4) (end 77.042 78.564) (width 0.2032) (layer B.Cu) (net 1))
 (segment (start 79.711 78.564) (end 79.975 78.3) (width 0.2032) (layer B.Cu) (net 1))
 (segment (start 77.142 78.564) (end 79.711 78.564) (width 0.2032) (layer B.Cu) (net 1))
 (segment (start 74.724 86.7033) (end 74.724 87.6565) (width 0.2032) (layer B.Cu) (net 1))
 (segment (start 74.724 83.1115) (end 74.724 86.7033) (width 0.2032) (layer B.Cu) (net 1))
 (segment (start 72.375 80.7625) (end 74.724 83.1115) (width 0.2032) (layer B.Cu) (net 1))
 (segment (start 72.375 80.175) (end 72.375 80.7625) (width 0.2032) (layer B.Cu) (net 1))
 (segment (start 78.575 105.375) (end 81.125 102.825) (width 0.2032) (layer B.Cu) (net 1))
 (segment (start 78.575 105.65) (end 78.575 105.375) (width 0.2032) (layer B.Cu) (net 1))
 (segment (start 80.2 107.275) (end 78.575 105.65) (width 0.2032) (layer B.Cu) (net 1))
 (segment (start 84.85 107.275) (end 80.2 107.275) (width 0.2032) (layer B.Cu) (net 1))
 (segment (start 86.2 100.325) (end 86.2 105.925) (width 0.2032) (layer B.Cu) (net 1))
 (segment (start 86.2 105.925) (end 84.85 107.275) (width 0.2032) (layer B.Cu) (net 1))
 (segment (start 68.425 90.725) (end 68.45 90.75) (width 0.2032) (layer F.Cu) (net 1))
 (segment (start 70.400601 93.933101) (end 70.624 94.1565) (width 0.2032) (layer B.Cu) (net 1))
 (segment (start 69.632719 93.933101) (end 70.400601 93.933101) (width 0.2032) (layer B.Cu) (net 1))
 (segment (start 73.124 100.0097) (end 73.124 99.0565) (width 0.2032) (layer B.Cu) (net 1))
 (segment (start 73.025599 100.108101) (end 73.124 100.0097) (width 0.2032) (layer B.Cu) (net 1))
 (via (at 72.675 82.525) (size 0.8) (drill 0.4) (layers F.Cu B.Cu) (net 1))
 (segment (start 72.375 80.175) (end 72.375 82.225) (width 0.2032) (layer B.Cu) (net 1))
 (segment (start 72.375 82.225) (end 72.675 82.525) (width 0.2032) (layer B.Cu) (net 1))
 (via (at 76.35 82.55) (size 0.8) (drill 0.4) (layers F.Cu B.Cu) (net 1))
 (segment (start 72.675 82.525) (end 76.325 82.525) (width 0.2032) (layer F.Cu) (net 1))
 (segment (start 76.325 82.525) (end 76.35 82.55) (width 0.2032) (layer F.Cu) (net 1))
 (segment (start 75.042 80.264) (end 74.942 80.264) (width 0.2032) (layer B.Cu) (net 1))
 (segment (start 76.35 81.572) (end 75.042 80.264) (width 0.2032) (layer B.Cu) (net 1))
 (segment (start 76.35 82.55) (end 76.35 81.572) (width 0.2032) (layer B.Cu) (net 1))
 (segment (start 82.024 88.8783) (end 82.024 89.3565) (width 0.2032) (layer B.Cu) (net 1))
 (segment (start 82.4898 88.4125) (end 82.024 88.8783) (width 0.2032) (layer B.Cu) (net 1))
 (segment (start 85.55 88.4125) (end 82.4898 88.4125) (width 0.2032) (layer B.Cu) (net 1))
 (segment (start 77.231 80.175) (end 77.142 80.264) (width 0.2032) (layer B.Cu) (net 3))
 (segment (start 79.975 80.175) (end 77.231 80.175) (width 0.2032) (layer B.Cu) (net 3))
 (segment (start 77.142 81.0672) (end 77.15 81.0752) (width 0.2032) (layer B.Cu) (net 3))
 (segment (start 77.142 80.264) (end 77.142 81.0672) (width 0.2032) (layer B.Cu) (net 3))
 (segment (start 77.15 81.0752) (end 77.15 84.4) (width 0.2032) (layer B.Cu) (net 3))
 (segment (start 76.324 85.226) (end 76.324 87.6565) (width 0.2032) (layer B.Cu) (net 3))
 (segment (start 77.15 84.4) (end 76.324 85.226) (width 0.2032) (layer B.Cu) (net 3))
 (segment (start 74.678 78.3) (end 74.942 78.564) (width 0.2032) (layer B.Cu) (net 4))
 (segment (start 72.375 78.3) (end 74.678 78.3) (width 0.2032) (layer B.Cu) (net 4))
 (segment (start 74.0388 78.564) (end 73.8 78.8028) (width 0.2032) (layer B.Cu) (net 4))
 (segment (start 74.942 78.564) (end 74.0388 78.564) (width 0.2032) (layer B.Cu) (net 4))
 (segment (start 75.524 86.7033) (end 75.524 87.6565) (width 0.2032) (layer B.Cu) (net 4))
 (segment (start 75.524 82.688882) (end 75.524 86.7033) (width 0.2032) (layer B.Cu) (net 4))
 (segment (start 73.8 80.964882) (end 75.524 82.688882) (width 0.2032) (layer B.Cu) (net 4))
 (segment (start 73.8 78.8028) (end 73.8 80.964882) (width 0.2032) (layer B.Cu) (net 4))
 (segment (start 99.875 95.60775) (end 100.23275 95.60775) (width 0.2032) (layer B.Cu) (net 10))
 (segment (start 52.35 77.166139) (end 52.387946 77.030624) (width 0.2032) (layer B.Cu) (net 12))
 (segment (start 52.35 80.478742) (end 52.35 77.166139) (width 0.2032) (layer B.Cu) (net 12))
 (segment (start 47.13 89.29) (end 47.13 85.698742) (width 0.2032) (layer B.Cu) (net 12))
 (segment (start 47.13 85.698742) (end 52.35 80.478742) (width 0.2032) (layer B.Cu) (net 12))
 (segment (start 53.15 78.3482) (end 53.15 77.02) (width 0.2032) (layer B.Cu) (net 23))
 (segment (start 53.15 82.7) (end 53.15 77.02) (width 0.2032) (layer B.Cu) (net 23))
 (segment (start 52 83.85) (end 53.15 82.7) (width 0.2032) (layer B.Cu) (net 23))
 (segment (start 52 86.3125) (end 53.375 87.6875) (width 0.2032) (layer B.Cu) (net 24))
 (segment (start 52 85.725) (end 52 86.3125) (width 0.2032) (layer B.Cu) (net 24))
 (segment (start 53.375 87.6875) (end 53.375 91.475) (width 0.2032) (layer B.Cu) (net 24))
 (segment (start 57.6565 95.7565) (end 70.624 95.7565) (width 0.2032) (layer B.Cu) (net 24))
 (segment (start 53.375 91.475) (end 57.6565 95.7565) (width 0.2032) (layer B.Cu) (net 24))
 (segment (start 55.05 86.425) (end 54.025 87.45) (width 0.2032) (layer B.Cu) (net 25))
 (segment (start 55.05 85.8375) (end 55.05 86.425) (width 0.2032) (layer B.Cu) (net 25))
 (segment (start 54.025 87.45) (end 54.025 91.275) (width 0.2032) (layer B.Cu) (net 25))
 (segment (start 57.7065 94.9565) (end 70.624 94.9565) (width 0.2032) (layer B.Cu) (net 25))
 (segment (start 54.025 91.275) (end 57.7065 94.9565) (width 0.2032) (layer B.Cu) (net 25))
 (segment (start 53.95 82.8625) (end 55.05 83.9625) (width 0.2032) (layer B.Cu) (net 26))
 (segment (start 53.95 77.02) (end 53.95 82.8625) (width 0.2032) (layer B.Cu) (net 26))
 (segment (start 62 83.2375) (end 63.0125 84.25) (width 0.2032) (layer B.Cu) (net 27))
 (segment (start 62 82.65) (end 62 83.2375) (width 0.2032) (layer B.Cu) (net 27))
 (segment (start 73.124 86.7033) (end 73.124 87.6565) (width 0.2032) (layer B.Cu) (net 27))
 (segment (start 73.124 85.949) (end 73.124 86.7033) (width 0.2032) (layer B.Cu) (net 27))
 (segment (start 71.425 84.25) (end 73.124 85.949) (width 0.2032) (layer B.Cu) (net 27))
 (segment (start 63.0125 84.25) (end 71.425 84.25) (width 0.2032) (layer B.Cu) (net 27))
 (segment (start 56.6 99.375) (end 57.7032 99.375) (width 0.2032) (layer B.Cu) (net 27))
 (via (at 60.625 98.1) (size 0.8) (drill 0.4) (layers F.Cu B.Cu) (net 27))
 (segment (start 56.6 99.375) (end 59.35 99.375) (width 0.2032) (layer B.Cu) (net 27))
 (segment (start 59.35 99.375) (end 60.625 98.1) (width 0.2032) (layer B.Cu) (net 27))
 (via (at 61.1 86.125) (size 0.8) (drill 0.4) (layers F.Cu B.Cu) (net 27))
 (segment (start 60.625 98.1) (end 61.1 97.625) (width 0.2032) (layer F.Cu) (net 27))
 (segment (start 61.1 97.625) (end 61.1 86.125) (width 0.2032) (layer F.Cu) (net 27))
 (segment (start 61.1 83.55) (end 62 82.65) (width 0.2032) (layer B.Cu) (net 27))
 (segment (start 61.1 86.125) (end 61.1 83.55) (width 0.2032) (layer B.Cu) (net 27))
 (segment (start 85.1065 97.3565) (end 82.024 97.3565) (width 0.2032) (layer B.Cu) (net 28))
 (segment (start 86.2 98.45) (end 85.1065 97.3565) (width 0.2032) (layer B.Cu) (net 28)))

